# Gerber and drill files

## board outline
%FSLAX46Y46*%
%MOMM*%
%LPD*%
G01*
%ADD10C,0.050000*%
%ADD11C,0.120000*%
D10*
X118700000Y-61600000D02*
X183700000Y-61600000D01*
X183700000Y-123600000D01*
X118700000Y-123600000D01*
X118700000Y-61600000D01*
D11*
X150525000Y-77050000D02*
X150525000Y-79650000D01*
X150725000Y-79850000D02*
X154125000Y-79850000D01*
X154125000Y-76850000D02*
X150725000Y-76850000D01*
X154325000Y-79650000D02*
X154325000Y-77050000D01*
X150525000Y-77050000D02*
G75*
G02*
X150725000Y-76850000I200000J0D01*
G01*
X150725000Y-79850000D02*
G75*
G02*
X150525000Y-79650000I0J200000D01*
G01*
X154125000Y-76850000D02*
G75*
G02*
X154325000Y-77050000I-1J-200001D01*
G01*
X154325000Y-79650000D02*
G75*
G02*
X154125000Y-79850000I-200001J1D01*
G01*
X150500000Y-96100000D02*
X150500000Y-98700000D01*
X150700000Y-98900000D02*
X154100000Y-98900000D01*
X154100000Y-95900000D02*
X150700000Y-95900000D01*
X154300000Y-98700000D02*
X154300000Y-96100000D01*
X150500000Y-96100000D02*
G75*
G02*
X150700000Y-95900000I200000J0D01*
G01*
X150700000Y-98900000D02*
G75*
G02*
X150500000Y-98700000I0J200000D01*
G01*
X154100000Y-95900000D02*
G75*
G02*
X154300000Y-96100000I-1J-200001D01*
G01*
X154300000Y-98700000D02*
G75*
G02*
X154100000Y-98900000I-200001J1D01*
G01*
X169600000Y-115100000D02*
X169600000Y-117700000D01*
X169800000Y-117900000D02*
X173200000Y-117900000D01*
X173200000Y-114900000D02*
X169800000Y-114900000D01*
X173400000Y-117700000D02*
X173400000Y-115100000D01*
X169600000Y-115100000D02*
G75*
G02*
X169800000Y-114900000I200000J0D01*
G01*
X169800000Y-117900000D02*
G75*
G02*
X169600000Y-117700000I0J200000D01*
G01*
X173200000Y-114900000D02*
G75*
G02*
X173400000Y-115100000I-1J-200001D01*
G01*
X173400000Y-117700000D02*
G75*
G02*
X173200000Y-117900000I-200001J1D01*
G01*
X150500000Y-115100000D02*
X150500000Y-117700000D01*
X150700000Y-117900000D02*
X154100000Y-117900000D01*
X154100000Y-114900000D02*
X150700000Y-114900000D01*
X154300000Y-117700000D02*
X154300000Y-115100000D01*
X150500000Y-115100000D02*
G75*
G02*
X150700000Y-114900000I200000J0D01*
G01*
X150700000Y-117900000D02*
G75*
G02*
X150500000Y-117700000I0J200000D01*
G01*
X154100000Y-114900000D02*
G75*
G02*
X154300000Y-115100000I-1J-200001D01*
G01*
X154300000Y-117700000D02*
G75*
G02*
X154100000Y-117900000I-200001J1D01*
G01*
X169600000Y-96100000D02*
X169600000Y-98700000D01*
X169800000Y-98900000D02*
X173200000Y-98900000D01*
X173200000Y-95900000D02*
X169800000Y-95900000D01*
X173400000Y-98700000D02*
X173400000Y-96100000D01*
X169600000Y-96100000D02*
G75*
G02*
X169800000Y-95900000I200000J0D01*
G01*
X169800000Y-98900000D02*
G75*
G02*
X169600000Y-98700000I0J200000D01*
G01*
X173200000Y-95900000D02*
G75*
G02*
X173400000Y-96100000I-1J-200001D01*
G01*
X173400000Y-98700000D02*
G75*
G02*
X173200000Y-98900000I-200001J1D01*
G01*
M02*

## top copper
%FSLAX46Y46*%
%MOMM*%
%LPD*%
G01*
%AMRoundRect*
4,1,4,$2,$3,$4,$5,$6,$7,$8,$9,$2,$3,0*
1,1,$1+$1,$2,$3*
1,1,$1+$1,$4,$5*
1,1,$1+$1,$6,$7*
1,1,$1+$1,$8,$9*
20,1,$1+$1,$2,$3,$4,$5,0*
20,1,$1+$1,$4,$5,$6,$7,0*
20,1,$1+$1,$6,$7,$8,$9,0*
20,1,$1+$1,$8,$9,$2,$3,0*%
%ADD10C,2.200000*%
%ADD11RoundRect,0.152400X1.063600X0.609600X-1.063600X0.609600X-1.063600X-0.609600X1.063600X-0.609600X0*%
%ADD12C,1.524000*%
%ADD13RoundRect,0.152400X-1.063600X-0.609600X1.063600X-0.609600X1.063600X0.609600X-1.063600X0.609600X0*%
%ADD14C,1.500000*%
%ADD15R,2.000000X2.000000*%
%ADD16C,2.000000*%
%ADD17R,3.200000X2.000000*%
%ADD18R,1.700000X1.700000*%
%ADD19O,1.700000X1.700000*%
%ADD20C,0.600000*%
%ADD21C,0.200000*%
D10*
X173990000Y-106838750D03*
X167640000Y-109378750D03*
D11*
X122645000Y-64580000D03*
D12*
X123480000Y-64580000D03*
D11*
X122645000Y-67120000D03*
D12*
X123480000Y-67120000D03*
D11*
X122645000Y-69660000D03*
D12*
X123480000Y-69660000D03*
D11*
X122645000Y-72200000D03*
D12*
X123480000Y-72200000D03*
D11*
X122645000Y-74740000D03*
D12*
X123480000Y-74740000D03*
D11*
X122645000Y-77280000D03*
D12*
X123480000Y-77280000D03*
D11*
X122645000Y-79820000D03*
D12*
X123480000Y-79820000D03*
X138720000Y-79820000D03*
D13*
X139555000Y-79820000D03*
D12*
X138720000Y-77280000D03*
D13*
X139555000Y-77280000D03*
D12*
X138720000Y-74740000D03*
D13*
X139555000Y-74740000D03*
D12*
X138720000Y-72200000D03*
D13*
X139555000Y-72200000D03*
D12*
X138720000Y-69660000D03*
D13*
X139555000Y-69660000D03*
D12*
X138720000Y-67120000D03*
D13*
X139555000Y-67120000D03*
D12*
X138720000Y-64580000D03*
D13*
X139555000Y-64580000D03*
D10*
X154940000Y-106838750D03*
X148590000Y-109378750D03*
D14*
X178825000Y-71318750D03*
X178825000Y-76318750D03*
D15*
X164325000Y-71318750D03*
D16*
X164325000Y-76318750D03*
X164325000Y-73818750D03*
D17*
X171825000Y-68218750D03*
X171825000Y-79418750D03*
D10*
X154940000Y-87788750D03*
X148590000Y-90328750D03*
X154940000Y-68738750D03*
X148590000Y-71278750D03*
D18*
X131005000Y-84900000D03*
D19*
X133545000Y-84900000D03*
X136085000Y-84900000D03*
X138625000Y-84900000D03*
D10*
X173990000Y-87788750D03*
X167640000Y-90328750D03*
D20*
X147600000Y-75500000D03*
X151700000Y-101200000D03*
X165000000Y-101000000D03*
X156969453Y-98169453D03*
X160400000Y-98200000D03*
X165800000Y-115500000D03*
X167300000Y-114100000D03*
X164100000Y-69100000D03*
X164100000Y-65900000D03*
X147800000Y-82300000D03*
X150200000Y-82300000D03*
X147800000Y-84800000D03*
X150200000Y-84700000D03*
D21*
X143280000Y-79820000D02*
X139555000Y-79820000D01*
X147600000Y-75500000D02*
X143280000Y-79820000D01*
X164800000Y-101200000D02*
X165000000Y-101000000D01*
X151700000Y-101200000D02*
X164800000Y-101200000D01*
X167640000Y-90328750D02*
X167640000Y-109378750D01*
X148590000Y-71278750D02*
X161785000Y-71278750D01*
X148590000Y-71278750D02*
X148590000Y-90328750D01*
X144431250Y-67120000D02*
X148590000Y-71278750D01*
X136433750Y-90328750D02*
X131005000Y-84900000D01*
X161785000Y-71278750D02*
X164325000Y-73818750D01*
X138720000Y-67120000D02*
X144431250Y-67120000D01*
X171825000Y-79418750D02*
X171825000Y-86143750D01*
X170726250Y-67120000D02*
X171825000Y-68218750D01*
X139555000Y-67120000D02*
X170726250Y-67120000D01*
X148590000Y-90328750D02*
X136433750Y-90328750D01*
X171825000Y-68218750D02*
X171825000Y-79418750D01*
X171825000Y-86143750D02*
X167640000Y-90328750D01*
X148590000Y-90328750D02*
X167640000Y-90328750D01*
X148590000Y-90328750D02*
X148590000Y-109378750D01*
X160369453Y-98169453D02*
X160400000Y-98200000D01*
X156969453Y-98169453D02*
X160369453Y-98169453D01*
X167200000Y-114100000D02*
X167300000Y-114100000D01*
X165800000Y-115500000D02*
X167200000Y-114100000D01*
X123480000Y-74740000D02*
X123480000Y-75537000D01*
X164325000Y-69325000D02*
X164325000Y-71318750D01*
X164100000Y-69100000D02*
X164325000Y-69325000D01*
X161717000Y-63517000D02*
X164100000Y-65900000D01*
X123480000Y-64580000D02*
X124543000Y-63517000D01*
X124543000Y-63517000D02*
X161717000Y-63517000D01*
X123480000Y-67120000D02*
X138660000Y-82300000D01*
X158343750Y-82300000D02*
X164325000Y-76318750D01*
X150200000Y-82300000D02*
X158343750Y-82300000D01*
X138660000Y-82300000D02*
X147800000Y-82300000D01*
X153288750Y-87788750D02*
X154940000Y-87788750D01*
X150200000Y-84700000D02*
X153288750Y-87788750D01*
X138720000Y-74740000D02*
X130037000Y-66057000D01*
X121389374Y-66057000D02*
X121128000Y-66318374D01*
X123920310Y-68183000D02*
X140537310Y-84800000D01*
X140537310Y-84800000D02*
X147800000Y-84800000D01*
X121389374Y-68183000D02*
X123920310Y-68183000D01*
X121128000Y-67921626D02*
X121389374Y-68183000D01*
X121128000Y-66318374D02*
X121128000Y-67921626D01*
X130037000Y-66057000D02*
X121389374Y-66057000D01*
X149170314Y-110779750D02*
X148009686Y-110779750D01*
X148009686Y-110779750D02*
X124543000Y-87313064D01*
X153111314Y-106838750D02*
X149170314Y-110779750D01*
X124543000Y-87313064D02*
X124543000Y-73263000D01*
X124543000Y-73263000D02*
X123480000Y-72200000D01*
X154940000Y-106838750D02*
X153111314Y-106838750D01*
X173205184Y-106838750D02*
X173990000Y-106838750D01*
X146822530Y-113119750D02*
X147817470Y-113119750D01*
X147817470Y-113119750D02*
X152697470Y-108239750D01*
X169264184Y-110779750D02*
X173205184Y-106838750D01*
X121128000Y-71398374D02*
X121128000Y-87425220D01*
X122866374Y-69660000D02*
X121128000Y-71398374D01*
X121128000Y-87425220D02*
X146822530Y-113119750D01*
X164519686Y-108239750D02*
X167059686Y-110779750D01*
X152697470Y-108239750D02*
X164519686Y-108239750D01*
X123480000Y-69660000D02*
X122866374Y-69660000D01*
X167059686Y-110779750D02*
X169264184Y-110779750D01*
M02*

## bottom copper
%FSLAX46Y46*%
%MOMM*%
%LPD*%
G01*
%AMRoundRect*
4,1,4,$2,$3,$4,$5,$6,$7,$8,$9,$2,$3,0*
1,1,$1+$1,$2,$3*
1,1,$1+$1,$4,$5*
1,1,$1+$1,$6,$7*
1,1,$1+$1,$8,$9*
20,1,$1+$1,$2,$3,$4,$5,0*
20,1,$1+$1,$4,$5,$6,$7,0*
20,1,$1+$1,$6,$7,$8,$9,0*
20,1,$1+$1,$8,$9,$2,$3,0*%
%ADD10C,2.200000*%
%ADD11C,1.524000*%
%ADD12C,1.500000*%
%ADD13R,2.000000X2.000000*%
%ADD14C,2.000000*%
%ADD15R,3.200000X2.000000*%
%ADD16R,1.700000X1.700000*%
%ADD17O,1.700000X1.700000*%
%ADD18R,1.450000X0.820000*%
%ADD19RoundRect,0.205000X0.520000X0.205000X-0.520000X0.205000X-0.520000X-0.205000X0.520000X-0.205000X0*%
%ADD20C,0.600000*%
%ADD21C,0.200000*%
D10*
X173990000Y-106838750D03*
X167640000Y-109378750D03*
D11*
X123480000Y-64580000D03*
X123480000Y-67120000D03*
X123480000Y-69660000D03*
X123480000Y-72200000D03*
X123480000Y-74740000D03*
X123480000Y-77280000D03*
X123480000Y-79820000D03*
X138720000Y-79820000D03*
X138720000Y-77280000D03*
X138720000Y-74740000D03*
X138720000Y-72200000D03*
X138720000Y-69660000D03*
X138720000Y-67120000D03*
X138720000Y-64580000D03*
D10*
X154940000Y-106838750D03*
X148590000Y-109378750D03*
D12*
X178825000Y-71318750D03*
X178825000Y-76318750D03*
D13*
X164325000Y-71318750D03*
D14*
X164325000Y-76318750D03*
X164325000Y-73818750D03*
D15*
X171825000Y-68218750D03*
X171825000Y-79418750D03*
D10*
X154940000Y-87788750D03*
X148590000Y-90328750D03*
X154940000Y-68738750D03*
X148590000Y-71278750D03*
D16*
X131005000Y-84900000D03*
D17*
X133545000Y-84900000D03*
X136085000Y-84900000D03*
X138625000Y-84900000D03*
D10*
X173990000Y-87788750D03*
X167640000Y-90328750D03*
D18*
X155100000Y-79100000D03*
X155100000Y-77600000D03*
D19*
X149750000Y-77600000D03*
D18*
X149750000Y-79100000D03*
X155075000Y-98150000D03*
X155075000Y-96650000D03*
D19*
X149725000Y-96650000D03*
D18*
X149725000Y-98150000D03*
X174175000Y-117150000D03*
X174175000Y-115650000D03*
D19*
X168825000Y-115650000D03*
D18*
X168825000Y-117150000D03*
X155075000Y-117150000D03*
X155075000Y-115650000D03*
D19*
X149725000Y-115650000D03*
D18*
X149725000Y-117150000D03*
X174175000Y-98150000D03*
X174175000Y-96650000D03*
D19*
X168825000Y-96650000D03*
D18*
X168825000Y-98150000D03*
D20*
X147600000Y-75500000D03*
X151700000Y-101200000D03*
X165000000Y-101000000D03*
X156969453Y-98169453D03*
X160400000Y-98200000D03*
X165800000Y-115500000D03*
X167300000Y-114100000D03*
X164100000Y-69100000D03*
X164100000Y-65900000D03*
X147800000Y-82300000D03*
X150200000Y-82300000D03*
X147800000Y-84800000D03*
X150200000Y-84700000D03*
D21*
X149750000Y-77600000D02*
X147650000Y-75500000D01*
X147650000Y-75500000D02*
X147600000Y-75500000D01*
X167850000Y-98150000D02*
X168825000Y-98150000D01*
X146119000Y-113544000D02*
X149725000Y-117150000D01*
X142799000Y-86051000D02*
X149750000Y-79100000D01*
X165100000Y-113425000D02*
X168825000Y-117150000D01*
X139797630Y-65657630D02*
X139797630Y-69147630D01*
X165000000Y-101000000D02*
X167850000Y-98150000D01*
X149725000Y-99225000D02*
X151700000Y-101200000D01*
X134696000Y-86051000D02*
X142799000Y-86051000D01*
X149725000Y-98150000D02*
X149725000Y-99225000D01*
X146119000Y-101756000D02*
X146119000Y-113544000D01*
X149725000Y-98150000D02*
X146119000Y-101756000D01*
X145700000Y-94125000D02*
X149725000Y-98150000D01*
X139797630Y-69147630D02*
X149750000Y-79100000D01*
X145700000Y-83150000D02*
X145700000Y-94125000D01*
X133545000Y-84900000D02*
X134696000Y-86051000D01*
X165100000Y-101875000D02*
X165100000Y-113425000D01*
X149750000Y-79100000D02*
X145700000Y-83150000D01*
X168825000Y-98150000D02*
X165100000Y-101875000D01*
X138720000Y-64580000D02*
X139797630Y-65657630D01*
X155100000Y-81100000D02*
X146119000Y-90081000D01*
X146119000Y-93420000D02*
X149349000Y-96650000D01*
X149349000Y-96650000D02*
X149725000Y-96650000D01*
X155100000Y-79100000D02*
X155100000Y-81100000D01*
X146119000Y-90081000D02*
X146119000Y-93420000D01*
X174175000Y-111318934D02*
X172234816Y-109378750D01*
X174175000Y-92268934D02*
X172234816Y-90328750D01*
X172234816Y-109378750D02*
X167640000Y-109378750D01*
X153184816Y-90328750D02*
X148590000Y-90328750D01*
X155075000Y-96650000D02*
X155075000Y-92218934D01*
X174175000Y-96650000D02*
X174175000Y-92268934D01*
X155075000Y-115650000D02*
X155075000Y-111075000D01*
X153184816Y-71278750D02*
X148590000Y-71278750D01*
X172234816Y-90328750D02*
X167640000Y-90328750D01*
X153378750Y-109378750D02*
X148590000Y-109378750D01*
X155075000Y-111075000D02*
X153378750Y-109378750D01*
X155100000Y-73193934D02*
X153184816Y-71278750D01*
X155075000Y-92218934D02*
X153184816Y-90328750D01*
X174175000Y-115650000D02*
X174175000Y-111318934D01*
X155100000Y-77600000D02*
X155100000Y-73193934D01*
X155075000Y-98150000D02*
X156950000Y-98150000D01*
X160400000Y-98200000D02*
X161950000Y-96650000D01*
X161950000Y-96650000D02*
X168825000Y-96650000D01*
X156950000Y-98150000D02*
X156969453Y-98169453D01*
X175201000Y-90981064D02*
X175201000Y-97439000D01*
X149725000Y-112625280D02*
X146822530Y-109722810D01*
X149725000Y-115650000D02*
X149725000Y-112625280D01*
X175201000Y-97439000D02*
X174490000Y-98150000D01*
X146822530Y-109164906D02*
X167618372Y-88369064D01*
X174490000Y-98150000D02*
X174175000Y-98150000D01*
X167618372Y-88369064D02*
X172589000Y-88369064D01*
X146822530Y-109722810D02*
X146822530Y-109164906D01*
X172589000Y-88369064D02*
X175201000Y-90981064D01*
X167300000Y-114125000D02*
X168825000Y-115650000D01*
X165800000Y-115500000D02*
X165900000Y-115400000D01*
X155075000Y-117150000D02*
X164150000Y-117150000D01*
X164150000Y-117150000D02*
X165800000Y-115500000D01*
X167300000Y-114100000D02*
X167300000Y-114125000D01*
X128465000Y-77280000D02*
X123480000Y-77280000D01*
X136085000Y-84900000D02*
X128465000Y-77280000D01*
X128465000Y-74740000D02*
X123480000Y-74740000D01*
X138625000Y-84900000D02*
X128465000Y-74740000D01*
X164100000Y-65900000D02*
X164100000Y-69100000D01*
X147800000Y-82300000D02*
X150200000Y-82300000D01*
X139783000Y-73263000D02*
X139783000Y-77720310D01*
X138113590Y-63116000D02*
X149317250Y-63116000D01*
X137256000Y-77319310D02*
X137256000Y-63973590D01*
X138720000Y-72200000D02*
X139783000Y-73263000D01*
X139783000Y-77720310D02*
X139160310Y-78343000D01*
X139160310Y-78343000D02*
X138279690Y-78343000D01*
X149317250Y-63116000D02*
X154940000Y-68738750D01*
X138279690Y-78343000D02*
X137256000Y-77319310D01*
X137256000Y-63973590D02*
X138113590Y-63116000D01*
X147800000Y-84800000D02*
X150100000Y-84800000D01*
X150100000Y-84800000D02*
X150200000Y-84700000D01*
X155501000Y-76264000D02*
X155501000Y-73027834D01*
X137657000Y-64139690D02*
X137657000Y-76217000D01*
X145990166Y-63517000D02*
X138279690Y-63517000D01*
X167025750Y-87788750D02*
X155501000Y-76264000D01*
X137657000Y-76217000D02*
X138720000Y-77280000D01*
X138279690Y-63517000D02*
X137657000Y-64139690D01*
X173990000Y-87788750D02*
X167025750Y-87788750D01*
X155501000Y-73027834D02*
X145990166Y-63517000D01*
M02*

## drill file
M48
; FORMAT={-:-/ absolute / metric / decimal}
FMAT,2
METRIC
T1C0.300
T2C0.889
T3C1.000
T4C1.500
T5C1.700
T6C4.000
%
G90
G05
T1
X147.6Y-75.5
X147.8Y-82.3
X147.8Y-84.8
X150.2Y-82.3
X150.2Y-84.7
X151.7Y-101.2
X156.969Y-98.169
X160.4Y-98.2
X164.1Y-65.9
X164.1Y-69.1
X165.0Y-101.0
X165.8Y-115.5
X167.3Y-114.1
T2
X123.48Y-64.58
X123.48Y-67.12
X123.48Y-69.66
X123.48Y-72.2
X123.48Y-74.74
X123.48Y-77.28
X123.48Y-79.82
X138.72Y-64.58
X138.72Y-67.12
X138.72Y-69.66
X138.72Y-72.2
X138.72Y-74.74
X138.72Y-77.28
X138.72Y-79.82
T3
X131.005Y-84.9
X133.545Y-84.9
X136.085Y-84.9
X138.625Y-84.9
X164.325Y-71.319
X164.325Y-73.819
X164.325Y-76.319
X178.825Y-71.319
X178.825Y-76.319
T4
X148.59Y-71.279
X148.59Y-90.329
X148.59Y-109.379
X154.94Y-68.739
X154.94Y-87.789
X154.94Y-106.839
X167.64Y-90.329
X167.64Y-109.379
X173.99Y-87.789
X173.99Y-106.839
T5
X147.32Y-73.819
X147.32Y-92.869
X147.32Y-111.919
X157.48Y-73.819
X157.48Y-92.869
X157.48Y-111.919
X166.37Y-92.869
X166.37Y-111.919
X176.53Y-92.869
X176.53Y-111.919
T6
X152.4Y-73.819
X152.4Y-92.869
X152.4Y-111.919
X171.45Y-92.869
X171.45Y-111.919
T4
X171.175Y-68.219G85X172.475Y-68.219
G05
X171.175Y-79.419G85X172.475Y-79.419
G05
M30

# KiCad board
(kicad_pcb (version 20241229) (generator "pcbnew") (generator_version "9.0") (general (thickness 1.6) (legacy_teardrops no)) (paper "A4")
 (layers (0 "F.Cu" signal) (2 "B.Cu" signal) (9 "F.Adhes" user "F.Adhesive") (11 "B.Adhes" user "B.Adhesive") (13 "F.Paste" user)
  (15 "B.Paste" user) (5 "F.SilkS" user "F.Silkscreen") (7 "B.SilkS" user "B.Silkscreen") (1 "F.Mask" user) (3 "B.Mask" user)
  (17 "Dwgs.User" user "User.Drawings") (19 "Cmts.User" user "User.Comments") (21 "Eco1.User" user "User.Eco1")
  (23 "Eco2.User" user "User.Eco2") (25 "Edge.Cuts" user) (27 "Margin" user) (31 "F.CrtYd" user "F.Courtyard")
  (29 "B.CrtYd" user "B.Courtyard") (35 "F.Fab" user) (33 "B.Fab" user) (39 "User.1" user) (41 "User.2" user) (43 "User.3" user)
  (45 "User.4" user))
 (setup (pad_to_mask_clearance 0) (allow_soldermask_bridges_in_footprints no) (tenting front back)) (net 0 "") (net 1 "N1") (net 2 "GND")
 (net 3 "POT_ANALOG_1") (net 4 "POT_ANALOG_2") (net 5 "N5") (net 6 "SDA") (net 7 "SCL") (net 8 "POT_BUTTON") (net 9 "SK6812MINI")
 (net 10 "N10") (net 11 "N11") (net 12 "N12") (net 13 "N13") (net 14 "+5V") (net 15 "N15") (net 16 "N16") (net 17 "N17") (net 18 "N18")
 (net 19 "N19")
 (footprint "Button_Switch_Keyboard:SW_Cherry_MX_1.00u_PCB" (layer "F.Cu") (at 173.99 106.83875)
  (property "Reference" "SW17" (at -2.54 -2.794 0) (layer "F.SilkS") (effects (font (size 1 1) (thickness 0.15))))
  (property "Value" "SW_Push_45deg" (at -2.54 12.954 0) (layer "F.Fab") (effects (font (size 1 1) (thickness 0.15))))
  (pad "" np_thru_hole circle (at -7.62 5.08) (size 1.7 1.7) (drill 1.7) (layers "*.Cu" "*.Mask"))
  (pad "" np_thru_hole circle (at -2.54 5.08) (size 4 4) (drill 4) (layers "*.Cu" "*.Mask"))
  (pad "" np_thru_hole circle (at 2.54 5.08) (size 1.7 1.7) (drill 1.7) (layers "*.Cu" "*.Mask"))
  (pad "1" thru_hole circle (at 0 0) (size 2.2 2.2) (drill 1.5) (layers "*.Cu" "*.Mask") (remove_unused_layers no) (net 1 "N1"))
  (pad "2" thru_hole circle (at -6.35 2.54) (size 2.2 2.2) (drill 1.5) (layers "*.Cu" "*.Mask") (remove_unused_layers no) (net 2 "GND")))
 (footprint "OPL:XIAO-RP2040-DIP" (layer "F.Cu") (at 131.1 72.2)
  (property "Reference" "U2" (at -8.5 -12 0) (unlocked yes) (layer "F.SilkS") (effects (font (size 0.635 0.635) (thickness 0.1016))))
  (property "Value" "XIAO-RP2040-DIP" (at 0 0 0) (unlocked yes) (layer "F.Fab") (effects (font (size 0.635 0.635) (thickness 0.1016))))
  (pad "1" smd roundrect (at -8.455 -7.62 180) (size 2.432 1.524) (layers "F.Cu" "F.Mask") (roundrect_rratio 0.1) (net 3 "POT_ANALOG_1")
   (thermal_bridge_angle 45))
  (pad "1" thru_hole circle (at -7.62 -7.62 180) (size 1.524 1.524) (drill 0.889) (layers "*.Cu" "*.Mask") (remove_unused_layers no)
   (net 3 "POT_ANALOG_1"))
  (pad "2" smd roundrect (at -8.455 -5.08 180) (size 2.432 1.524) (layers "F.Cu" "F.Mask") (roundrect_rratio 0.1) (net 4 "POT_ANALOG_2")
   (thermal_bridge_angle 45))
  (pad "2" thru_hole circle (at -7.62 -5.08 180) (size 1.524 1.524) (drill 0.889) (layers "*.Cu" "*.Mask") (remove_unused_layers no)
   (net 4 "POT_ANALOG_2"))
  (pad "3" smd roundrect (at -8.455 -2.54 180) (size 2.432 1.524) (layers "F.Cu" "F.Mask") (roundrect_rratio 0.1) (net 1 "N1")
   (thermal_bridge_angle 45))
  (pad "3" thru_hole circle (at -7.62 -2.54 180) (size 1.524 1.524) (drill 0.889) (layers "*.Cu" "*.Mask") (remove_unused_layers no)
   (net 1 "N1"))
  (pad "4" smd roundrect (at -8.455 0 180) (size 2.432 1.524) (layers "F.Cu" "F.Mask") (roundrect_rratio 0.1) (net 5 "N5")
   (thermal_bridge_angle 45))
  (pad "4" thru_hole circle (at -7.62 0 180) (size 1.524 1.524) (drill 0.889) (layers "*.Cu" "*.Mask") (remove_unused_layers no)
   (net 5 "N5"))
  (pad "5" smd roundrect (at -8.455 2.54 180) (size 2.432 1.524) (layers "F.Cu" "F.Mask") (roundrect_rratio 0.1) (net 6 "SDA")
   (thermal_bridge_angle 45))
  (pad "5" thru_hole circle (at -7.62 2.54 180) (size 1.524 1.524) (drill 0.889) (layers "*.Cu" "*.Mask") (remove_unused_layers no)
   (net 6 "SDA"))
  (pad "6" smd roundrect (at -8.455 5.08 180) (size 2.432 1.524) (layers "F.Cu" "F.Mask") (roundrect_rratio 0.1) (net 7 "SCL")
   (thermal_bridge_angle 45))
  (pad "6" thru_hole circle (at -7.62 5.08 180) (size 1.524 1.524) (drill 0.889) (layers "*.Cu" "*.Mask") (remove_unused_layers no)
   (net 7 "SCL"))
  (pad "7" smd roundrect (at -8.455 7.62 180) (size 2.432 1.524) (layers "F.Cu" "F.Mask") (roundrect_rratio 0.1) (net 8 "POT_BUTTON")
   (thermal_bridge_angle 45))
  (pad "7" thru_hole circle (at -7.62 7.62 180) (size 1.524 1.524) (drill 0.889) (layers "*.Cu" "*.Mask") (remove_unused_layers no)
   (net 8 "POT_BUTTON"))
  (pad "8" thru_hole circle (at 7.62 7.62) (size 1.524 1.524) (drill 0.889) (layers "*.Cu" "*.Mask") (remove_unused_layers no)
   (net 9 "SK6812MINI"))
  (pad "8" smd roundrect (at 8.455 7.62) (size 2.432 1.524) (layers "F.Cu" "F.Mask") (roundrect_rratio 0.1) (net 9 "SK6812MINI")
   (thermal_bridge_angle 45))
  (pad "9" thru_hole circle (at 7.62 5.08) (size 1.524 1.524) (drill 0.889) (layers "*.Cu" "*.Mask") (remove_unused_layers no)
   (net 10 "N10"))
  (pad "9" smd roundrect (at 8.455 5.08) (size 2.432 1.524) (layers "F.Cu" "F.Mask") (roundrect_rratio 0.1) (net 10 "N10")
   (thermal_bridge_angle 45))
  (pad "10" thru_hole circle (at 7.62 2.54) (size 1.524 1.524) (drill 0.889) (layers "*.Cu" "*.Mask") (remove_unused_layers no)
   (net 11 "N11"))
  (pad "10" smd roundrect (at 8.455 2.54) (size 2.432 1.524) (layers "F.Cu" "F.Mask") (roundrect_rratio 0.1) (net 11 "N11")
   (thermal_bridge_angle 45))
  (pad "11" thru_hole circle (at 7.62 0) (size 1.524 1.524) (drill 0.889) (layers "*.Cu" "*.Mask") (remove_unused_layers no) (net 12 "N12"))
  (pad "11" smd roundrect (at 8.455 0) (size 2.432 1.524) (layers "F.Cu" "F.Mask") (roundrect_rratio 0.1) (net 12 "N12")
   (thermal_bridge_angle 45))
  (pad "12" thru_hole circle (at 7.62 -2.54) (size 1.524 1.524) (drill 0.889) (layers "*.Cu" "*.Mask") (remove_unused_layers no)
   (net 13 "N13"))
  (pad "12" smd roundrect (at 8.455 -2.54) (size 2.432 1.524) (layers "F.Cu" "F.Mask") (roundrect_rratio 0.1) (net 13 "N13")
   (thermal_bridge_angle 45))
  (pad "13" thru_hole circle (at 7.62 -5.08) (size 1.524 1.524) (drill 0.889) (layers "*.Cu" "*.Mask") (remove_unused_layers no)
   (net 2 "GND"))
  (pad "13" smd roundrect (at 8.455 -5.08) (size 2.432 1.524) (layers "F.Cu" "F.Mask") (roundrect_rratio 0.1) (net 2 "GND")
   (thermal_bridge_angle 45))
  (pad "14" thru_hole circle (at 7.62 -7.62) (size 1.524 1.524) (drill 0.889) (layers "*.Cu" "*.Mask") (remove_unused_layers no)
   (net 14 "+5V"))
  (pad "14" smd roundrect (at 8.455 -7.62) (size 2.432 1.524) (layers "F.Cu" "F.Mask") (roundrect_rratio 0.1) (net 14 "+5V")
   (thermal_bridge_angle 45)))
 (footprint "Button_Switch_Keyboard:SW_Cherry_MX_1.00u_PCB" (layer "F.Cu") (at 154.94 106.83875)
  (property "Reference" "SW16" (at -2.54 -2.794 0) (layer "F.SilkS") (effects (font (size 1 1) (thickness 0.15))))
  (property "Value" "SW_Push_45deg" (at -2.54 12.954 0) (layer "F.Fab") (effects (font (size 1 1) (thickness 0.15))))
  (pad "" np_thru_hole circle (at -7.62 5.08) (size 1.7 1.7) (drill 1.7) (layers "*.Cu" "*.Mask"))
  (pad "" np_thru_hole circle (at -2.54 5.08) (size 4 4) (drill 4) (layers "*.Cu" "*.Mask"))
  (pad "" np_thru_hole circle (at 2.54 5.08) (size 1.7 1.7) (drill 1.7) (layers "*.Cu" "*.Mask"))
  (pad "1" thru_hole circle (at 0 0) (size 2.2 2.2) (drill 1.5) (layers "*.Cu" "*.Mask") (remove_unused_layers no) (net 5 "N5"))
  (pad "2" thru_hole circle (at -6.35 2.54) (size 2.2 2.2) (drill 1.5) (layers "*.Cu" "*.Mask") (remove_unused_layers no) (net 2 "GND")))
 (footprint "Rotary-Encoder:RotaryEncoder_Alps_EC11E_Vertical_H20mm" (layer "F.Cu") (at 164.325 71.31875)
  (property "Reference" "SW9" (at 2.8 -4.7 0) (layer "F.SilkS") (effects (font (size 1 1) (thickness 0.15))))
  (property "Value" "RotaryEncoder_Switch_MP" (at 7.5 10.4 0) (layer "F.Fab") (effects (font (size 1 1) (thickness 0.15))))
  (pad "" thru_hole circle (at 14.5 0) (size 1.5 1.5) (drill 1) (layers "*.Cu" "*.Mask") (remove_unused_layers no))
  (pad "" thru_hole circle (at 14.5 5) (size 1.5 1.5) (drill 1) (layers "*.Cu" "*.Mask") (remove_unused_layers no))
  (pad "A" thru_hole rect (at 0 0) (size 2 2) (drill 1) (layers "*.Cu" "*.Mask") (remove_unused_layers no) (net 3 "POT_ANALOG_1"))
  (pad "B" thru_hole circle (at 0 5) (size 2 2) (drill 1) (layers "*.Cu" "*.Mask") (remove_unused_layers no) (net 4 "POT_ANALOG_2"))
  (pad "C" thru_hole circle (at 0 2.5) (size 2 2) (drill 1) (layers "*.Cu" "*.Mask") (remove_unused_layers no) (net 2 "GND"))
  (pad "MP" thru_hole rect (at 7.5 -3.1) (size 3.2 2) (drill oval 2.8 1.5) (layers "*.Cu" "*.Mask") (remove_unused_layers no) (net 2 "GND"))
  (pad "MP" thru_hole rect (at 7.5 8.1) (size 3.2 2) (drill oval 2.8 1.5) (layers "*.Cu" "*.Mask") (remove_unused_layers no) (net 2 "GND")))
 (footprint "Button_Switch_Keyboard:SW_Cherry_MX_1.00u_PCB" (layer "F.Cu") (at 154.94 87.78875)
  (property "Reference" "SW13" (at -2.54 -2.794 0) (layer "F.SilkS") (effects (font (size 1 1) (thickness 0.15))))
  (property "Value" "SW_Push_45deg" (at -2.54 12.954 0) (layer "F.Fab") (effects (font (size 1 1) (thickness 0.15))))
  (pad "" np_thru_hole circle (at -7.62 5.08) (size 1.7 1.7) (drill 1.7) (layers "*.Cu" "*.Mask"))
  (pad "" np_thru_hole circle (at -2.54 5.08) (size 4 4) (drill 4) (layers "*.Cu" "*.Mask"))
  (pad "" np_thru_hole circle (at 2.54 5.08) (size 1.7 1.7) (drill 1.7) (layers "*.Cu" "*.Mask"))
  (pad "1" thru_hole circle (at 0 0) (size 2.2 2.2) (drill 1.5) (layers "*.Cu" "*.Mask") (remove_unused_layers no) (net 11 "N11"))
  (pad "2" thru_hole circle (at -6.35 2.54) (size 2.2 2.2) (drill 1.5) (layers "*.Cu" "*.Mask") (remove_unused_layers no) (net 2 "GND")))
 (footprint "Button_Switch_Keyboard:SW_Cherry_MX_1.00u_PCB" (layer "F.Cu") (at 154.94 68.73875)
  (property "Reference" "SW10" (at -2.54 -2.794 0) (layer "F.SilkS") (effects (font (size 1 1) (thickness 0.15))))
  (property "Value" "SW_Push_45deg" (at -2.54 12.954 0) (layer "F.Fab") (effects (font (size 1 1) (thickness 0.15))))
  (pad "" np_thru_hole circle (at -7.62 5.08) (size 1.7 1.7) (drill 1.7) (layers "*.Cu" "*.Mask"))
  (pad "" np_thru_hole circle (at -2.54 5.08) (size 4 4) (drill 4) (layers "*.Cu" "*.Mask"))
  (pad "" np_thru_hole circle (at 2.54 5.08) (size 1.7 1.7) (drill 1.7) (layers "*.Cu" "*.Mask"))
  (pad "1" thru_hole circle (at 0 0) (size 2.2 2.2) (drill 1.5) (layers "*.Cu" "*.Mask") (remove_unused_layers no) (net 12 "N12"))
  (pad "2" thru_hole circle (at -6.35 2.54) (size 2.2 2.2) (drill 1.5) (layers "*.Cu" "*.Mask") (remove_unused_layers no) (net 2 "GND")))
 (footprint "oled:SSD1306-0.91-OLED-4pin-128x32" (layer "F.Cu") (at 128.815 121.4 90)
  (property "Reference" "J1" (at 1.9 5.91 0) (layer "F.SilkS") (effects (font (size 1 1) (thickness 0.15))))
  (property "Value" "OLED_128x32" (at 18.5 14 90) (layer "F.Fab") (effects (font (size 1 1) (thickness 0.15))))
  (pad "1" thru_hole rect (at 36.5 2.19 90) (size 1.7 1.7) (drill 1) (layers "*.Cu" "*.Mask") (remove_unused_layers no) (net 2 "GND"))
  (pad "2" thru_hole oval (at 36.5 4.73 90) (size 1.7 1.7) (drill 1) (layers "*.Cu" "*.Mask") (remove_unused_layers no) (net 14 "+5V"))
  (pad "3" thru_hole oval (at 36.5 7.27 90) (size 1.7 1.7) (drill 1) (layers "*.Cu" "*.Mask") (remove_unused_layers no) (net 7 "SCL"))
  (pad "4" thru_hole oval (at 36.5 9.81 90) (size 1.7 1.7) (drill 1) (layers "*.Cu" "*.Mask") (remove_unused_layers no) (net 6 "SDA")))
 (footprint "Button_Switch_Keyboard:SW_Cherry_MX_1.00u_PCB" (layer "F.Cu") (at 173.99 87.78875)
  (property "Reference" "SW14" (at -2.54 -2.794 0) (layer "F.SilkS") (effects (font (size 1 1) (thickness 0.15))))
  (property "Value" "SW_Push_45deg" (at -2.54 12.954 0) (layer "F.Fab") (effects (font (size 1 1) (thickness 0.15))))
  (pad "" np_thru_hole circle (at -7.62 5.08) (size 1.7 1.7) (drill 1.7) (layers "*.Cu" "*.Mask"))
  (pad "" np_thru_hole circle (at -2.54 5.08) (size 4 4) (drill 4) (layers "*.Cu" "*.Mask"))
  (pad "" np_thru_hole circle (at 2.54 5.08) (size 1.7 1.7) (drill 1.7) (layers "*.Cu" "*.Mask"))
  (pad "1" thru_hole circle (at 0 0) (size 2.2 2.2) (drill 1.5) (layers "*.Cu" "*.Mask") (remove_unused_layers no) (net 10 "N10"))
  (pad "2" thru_hole circle (at -6.35 2.54) (size 2.2 2.2) (drill 1.5) (layers "*.Cu" "*.Mask") (remove_unused_layers no) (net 2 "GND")))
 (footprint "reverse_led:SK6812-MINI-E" (layer "B.Cu") (at 152.425 78.35 180)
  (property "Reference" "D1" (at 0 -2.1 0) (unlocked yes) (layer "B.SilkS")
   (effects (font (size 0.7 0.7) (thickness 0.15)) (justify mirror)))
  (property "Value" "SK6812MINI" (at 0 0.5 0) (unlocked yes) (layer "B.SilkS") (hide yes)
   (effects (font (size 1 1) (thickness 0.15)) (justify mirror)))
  (fp_line (start 1.9 1.3) (end 1.9 -1.3) (stroke (width 0.12) (type solid)) (layer "Edge.Cuts"))
  (fp_line (start 1.7 -1.5) (end -1.7 -1.5) (stroke (width 0.12) (type solid)) (layer "Edge.Cuts"))
  (fp_line (start -1.7 1.5) (end 1.7 1.5) (stroke (width 0.12) (type solid)) (layer "Edge.Cuts"))
  (fp_line (start -1.9 -1.3) (end -1.9 1.3) (stroke (width 0.12) (type solid)) (layer "Edge.Cuts"))
  (fp_arc (start 1.9 1.3) (mid 1.841421 1.441421) (end 1.7 1.5) (stroke (width 0.12) (type solid)) (layer "Edge.Cuts"))
  (fp_arc (start 1.7 -1.5) (mid 1.841421 -1.441421) (end 1.9 -1.3) (stroke (width 0.12) (type solid)) (layer "Edge.Cuts"))
  (fp_arc (start -1.7 1.5) (mid -1.841421 1.441421) (end -1.9 1.3) (stroke (width 0.12) (type solid)) (layer "Edge.Cuts"))
  (fp_arc (start -1.9 -1.3) (mid -1.841421 -1.441421) (end -1.7 -1.5) (stroke (width 0.12) (type solid)) (layer "Edge.Cuts"))
  (pad "1" smd rect (at -2.675 -0.75 180) (size 1.45 0.82) (layers "B.Cu" "B.Mask" "B.Paste") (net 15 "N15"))
  (pad "2" smd rect (at -2.675 0.75 180) (size 1.45 0.82) (layers "B.Cu" "B.Mask" "B.Paste") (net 2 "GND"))
  (pad "3" smd roundrect (at 2.675 0.75 180) (size 1.45 0.82) (layers "B.Cu" "B.Mask" "B.Paste") (roundrect_rratio 0.25)
   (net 9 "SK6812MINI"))
  (pad "4" smd rect (at 2.675 -0.75 180) (size 1.45 0.82) (layers "B.Cu" "B.Mask" "B.Paste") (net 14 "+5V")))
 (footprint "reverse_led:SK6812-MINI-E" (layer "B.Cu") (at 152.4 97.4 180)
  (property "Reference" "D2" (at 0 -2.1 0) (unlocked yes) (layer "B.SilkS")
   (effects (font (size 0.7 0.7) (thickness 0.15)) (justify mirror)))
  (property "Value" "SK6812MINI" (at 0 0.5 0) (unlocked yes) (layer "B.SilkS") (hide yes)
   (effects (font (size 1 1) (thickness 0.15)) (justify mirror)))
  (fp_line (start 1.9 1.3) (end 1.9 -1.3) (stroke (width 0.12) (type solid)) (layer "Edge.Cuts"))
  (fp_line (start 1.7 -1.5) (end -1.7 -1.5) (stroke (width 0.12) (type solid)) (layer "Edge.Cuts"))
  (fp_line (start -1.7 1.5) (end 1.7 1.5) (stroke (width 0.12) (type solid)) (layer "Edge.Cuts"))
  (fp_line (start -1.9 -1.3) (end -1.9 1.3) (stroke (width 0.12) (type solid)) (layer "Edge.Cuts"))
  (fp_arc (start 1.9 1.3) (mid 1.841421 1.441421) (end 1.7 1.5) (stroke (width 0.12) (type solid)) (layer "Edge.Cuts"))
  (fp_arc (start 1.7 -1.5) (mid 1.841421 -1.441421) (end 1.9 -1.3) (stroke (width 0.12) (type solid)) (layer "Edge.Cuts"))
  (fp_arc (start -1.7 1.5) (mid -1.841421 1.441421) (end -1.9 1.3) (stroke (width 0.12) (type solid)) (layer "Edge.Cuts"))
  (fp_arc (start -1.9 -1.3) (mid -1.841421 -1.441421) (end -1.7 -1.5) (stroke (width 0.12) (type solid)) (layer "Edge.Cuts"))
  (pad "1" smd rect (at -2.675 -0.75 180) (size 1.45 0.82) (layers "B.Cu" "B.Mask" "B.Paste") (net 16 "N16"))
  (pad "2" smd rect (at -2.675 0.75 180) (size 1.45 0.82) (layers "B.Cu" "B.Mask" "B.Paste") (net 2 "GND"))
  (pad "3" smd roundrect (at 2.675 0.75 180) (size 1.45 0.82) (layers "B.Cu" "B.Mask" "B.Paste") (roundrect_rratio 0.25) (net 15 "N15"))
  (pad "4" smd rect (at 2.675 -0.75 180) (size 1.45 0.82) (layers "B.Cu" "B.Mask" "B.Paste") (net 14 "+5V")))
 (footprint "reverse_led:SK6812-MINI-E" (layer "B.Cu") (at 171.5 116.4 180)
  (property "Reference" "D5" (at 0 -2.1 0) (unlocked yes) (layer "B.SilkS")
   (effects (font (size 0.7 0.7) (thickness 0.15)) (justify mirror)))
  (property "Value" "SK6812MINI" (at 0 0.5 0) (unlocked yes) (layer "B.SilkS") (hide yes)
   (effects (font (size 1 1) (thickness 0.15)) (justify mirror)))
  (fp_line (start 1.9 1.3) (end 1.9 -1.3) (stroke (width 0.12) (type solid)) (layer "Edge.Cuts"))
  (fp_line (start 1.7 -1.5) (end -1.7 -1.5) (stroke (width 0.12) (type solid)) (layer "Edge.Cuts"))
  (fp_line (start -1.7 1.5) (end 1.7 1.5) (stroke (width 0.12) (type solid)) (layer "Edge.Cuts"))
  (fp_line (start -1.9 -1.3) (end -1.9 1.3) (stroke (width 0.12) (type solid)) (layer "Edge.Cuts"))
  (fp_arc (start 1.9 1.3) (mid 1.841421 1.441421) (end 1.7 1.5) (stroke (width 0.12) (type solid)) (layer "Edge.Cuts"))
  (fp_arc (start 1.7 -1.5) (mid 1.841421 -1.441421) (end 1.9 -1.3) (stroke (width 0.12) (type solid)) (layer "Edge.Cuts"))
  (fp_arc (start -1.7 1.5) (mid -1.841421 1.441421) (end -1.9 1.3) (stroke (width 0.12) (type solid)) (layer "Edge.Cuts"))
  (fp_arc (start -1.9 -1.3) (mid -1.841421 -1.441421) (end -1.7 -1.5) (stroke (width 0.12) (type solid)) (layer "Edge.Cuts"))
  (pad "1" smd rect (at -2.675 -0.75 180) (size 1.45 0.82) (layers "B.Cu" "B.Mask" "B.Paste") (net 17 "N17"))
  (pad "2" smd rect (at -2.675 0.75 180) (size 1.45 0.82) (layers "B.Cu" "B.Mask" "B.Paste") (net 2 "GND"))
  (pad "3" smd roundrect (at 2.675 0.75 180) (size 1.45 0.82) (layers "B.Cu" "B.Mask" "B.Paste") (roundrect_rratio 0.25) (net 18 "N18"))
  (pad "4" smd rect (at 2.675 -0.75 180) (size 1.45 0.82) (layers "B.Cu" "B.Mask" "B.Paste") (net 14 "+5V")))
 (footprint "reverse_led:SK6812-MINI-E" (layer "B.Cu") (at 152.4 116.4 180)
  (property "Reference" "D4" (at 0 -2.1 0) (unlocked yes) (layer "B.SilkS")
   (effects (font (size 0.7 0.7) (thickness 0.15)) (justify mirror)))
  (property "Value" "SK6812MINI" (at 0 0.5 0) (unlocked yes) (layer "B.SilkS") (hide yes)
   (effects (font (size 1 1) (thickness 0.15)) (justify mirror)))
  (fp_line (start 1.9 1.3) (end 1.9 -1.3) (stroke (width 0.12) (type solid)) (layer "Edge.Cuts"))
  (fp_line (start 1.7 -1.5) (end -1.7 -1.5) (stroke (width 0.12) (type solid)) (layer "Edge.Cuts"))
  (fp_line (start -1.7 1.5) (end 1.7 1.5) (stroke (width 0.12) (type solid)) (layer "Edge.Cuts"))
  (fp_line (start -1.9 -1.3) (end -1.9 1.3) (stroke (width 0.12) (type solid)) (layer "Edge.Cuts"))
  (fp_arc (start 1.9 1.3) (mid 1.841421 1.441421) (end 1.7 1.5) (stroke (width 0.12) (type solid)) (layer "Edge.Cuts"))
  (fp_arc (start 1.7 -1.5) (mid 1.841421 -1.441421) (end 1.9 -1.3) (stroke (width 0.12) (type solid)) (layer "Edge.Cuts"))
  (fp_arc (start -1.7 1.5) (mid -1.841421 1.441421) (end -1.9 1.3) (stroke (width 0.12) (type solid)) (layer "Edge.Cuts"))
  (fp_arc (start -1.9 -1.3) (mid -1.841421 -1.441421) (end -1.7 -1.5) (stroke (width 0.12) (type solid)) (layer "Edge.Cuts"))
  (pad "1" smd rect (at -2.675 -0.75 180) (size 1.45 0.82) (layers "B.Cu" "B.Mask" "B.Paste") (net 18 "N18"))
  (pad "2" smd rect (at -2.675 0.75 180) (size 1.45 0.82) (layers "B.Cu" "B.Mask" "B.Paste") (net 2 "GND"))
  (pad "3" smd roundrect (at 2.675 0.75 180) (size 1.45 0.82) (layers "B.Cu" "B.Mask" "B.Paste") (roundrect_rratio 0.25) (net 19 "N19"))
  (pad "4" smd rect (at 2.675 -0.75 180) (size 1.45 0.82) (layers "B.Cu" "B.Mask" "B.Paste") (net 14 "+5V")))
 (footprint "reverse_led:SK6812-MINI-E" (layer "B.Cu") (at 171.5 97.4 180)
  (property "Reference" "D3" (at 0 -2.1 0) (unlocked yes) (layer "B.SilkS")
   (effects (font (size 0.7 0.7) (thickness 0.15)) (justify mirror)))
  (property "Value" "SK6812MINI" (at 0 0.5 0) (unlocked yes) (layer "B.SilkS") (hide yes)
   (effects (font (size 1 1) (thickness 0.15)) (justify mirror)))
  (fp_line (start 1.9 1.3) (end 1.9 -1.3) (stroke (width 0.12) (type solid)) (layer "Edge.Cuts"))
  (fp_line (start 1.7 -1.5) (end -1.7 -1.5) (stroke (width 0.12) (type solid)) (layer "Edge.Cuts"))
  (fp_line (start -1.7 1.5) (end 1.7 1.5) (stroke (width 0.12) (type solid)) (layer "Edge.Cuts"))
  (fp_line (start -1.9 -1.3) (end -1.9 1.3) (stroke (width 0.12) (type solid)) (layer "Edge.Cuts"))
  (fp_arc (start 1.9 1.3) (mid 1.841421 1.441421) (end 1.7 1.5) (stroke (width 0.12) (type solid)) (layer "Edge.Cuts"))
  (fp_arc (start 1.7 -1.5) (mid 1.841421 -1.441421) (end 1.9 -1.3) (stroke (width 0.12) (type solid)) (layer "Edge.Cuts"))
  (fp_arc (start -1.7 1.5) (mid -1.841421 1.441421) (end -1.9 1.3) (stroke (width 0.12) (type solid)) (layer "Edge.Cuts"))
  (fp_arc (start -1.9 -1.3) (mid -1.841421 -1.441421) (end -1.7 -1.5) (stroke (width 0.12) (type solid)) (layer "Edge.Cuts"))
  (pad "1" smd rect (at -2.675 -0.75 180) (size 1.45 0.82) (layers "B.Cu" "B.Mask" "B.Paste") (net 19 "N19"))
  (pad "2" smd rect (at -2.675 0.75 180) (size 1.45 0.82) (layers "B.Cu" "B.Mask" "B.Paste") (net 2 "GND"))
  (pad "3" smd roundrect (at 2.675 0.75 180) (size 1.45 0.82) (layers "B.Cu" "B.Mask" "B.Paste") (roundrect_rratio 0.25) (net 16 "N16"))
  (pad "4" smd rect (at 2.675 -0.75 180) (size 1.45 0.82) (layers "B.Cu" "B.Mask" "B.Paste") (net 14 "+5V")))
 (gr_rect (start 118.7 61.6) (end 183.7 123.6) (stroke (width 0.05) (type solid)) (fill no) (layer "Edge.Cuts"))
 (segment (start 143.28 79.82) (end 139.555 79.82) (width 0.2) (layer "F.Cu") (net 9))
 (segment (start 147.6 75.5) (end 143.28 79.82) (width 0.2) (layer "F.Cu") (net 9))
 (via (at 147.6 75.5) (size 0.6) (drill 0.3) (layers "F.Cu" "B.Cu") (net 9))
 (segment (start 149.75 77.6) (end 147.65 75.5) (width 0.2) (layer "B.Cu") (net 9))
 (segment (start 147.65 75.5) (end 147.6 75.5) (width 0.2) (layer "B.Cu") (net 9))
 (segment (start 164.8 101.2) (end 165 101) (width 0.2) (layer "F.Cu") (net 14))
 (segment (start 151.7 101.2) (end 164.8 101.2) (width 0.2) (layer "F.Cu") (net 14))
 (via (at 151.7 101.2) (size 0.6) (drill 0.3) (layers "F.Cu" "B.Cu") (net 14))
 (via (at 165 101) (size 0.6) (drill 0.3) (layers "F.Cu" "B.Cu") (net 14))
 (segment (start 167.85 98.15) (end 168.825 98.15) (width 0.2) (layer "B.Cu") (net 14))
 (segment (start 146.119 113.544) (end 149.725 117.15) (width 0.2) (layer "B.Cu") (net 14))
 (segment (start 142.799 86.051) (end 149.75 79.1) (width 0.2) (layer "B.Cu") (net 14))
 (segment (start 165.1 113.425) (end 168.825 117.15) (width 0.2) (layer "B.Cu") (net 14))
 (segment (start 139.79763 65.65763) (end 139.79763 69.14763) (width 0.2) (layer "B.Cu") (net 14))
 (segment (start 165 101) (end 167.85 98.15) (width 0.2) (layer "B.Cu") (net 14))
 (segment (start 149.725 99.225) (end 151.7 101.2) (width 0.2) (layer "B.Cu") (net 14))
 (segment (start 134.696 86.051) (end 142.799 86.051) (width 0.2) (layer "B.Cu") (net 14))
 (segment (start 149.725 98.15) (end 149.725 99.225) (width 0.2) (layer "B.Cu") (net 14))
 (segment (start 146.119 101.756) (end 146.119 113.544) (width 0.2) (layer "B.Cu") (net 14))
 (segment (start 149.725 98.15) (end 146.119 101.756) (width 0.2) (layer "B.Cu") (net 14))
 (segment (start 145.7 94.125) (end 149.725 98.15) (width 0.2) (layer "B.Cu") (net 14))
 (segment (start 139.79763 69.14763) (end 149.75 79.1) (width 0.2) (layer "B.Cu") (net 14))
 (segment (start 145.7 83.15) (end 145.7 94.125) (width 0.2) (layer "B.Cu") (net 14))
 (segment (start 133.545 84.9) (end 134.696 86.051) (width 0.2) (layer "B.Cu") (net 14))
 (segment (start 165.1 101.875) (end 165.1 113.425) (width 0.2) (layer "B.Cu") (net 14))
 (segment (start 149.75 79.1) (end 145.7 83.15) (width 0.2) (layer "B.Cu") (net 14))
 (segment (start 168.825 98.15) (end 165.1 101.875) (width 0.2) (layer "B.Cu") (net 14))
 (segment (start 138.72 64.58) (end 139.79763 65.65763) (width 0.2) (layer "B.Cu") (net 14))
 (segment (start 155.1 81.1) (end 146.119 90.081) (width 0.2) (layer "B.Cu") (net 15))
 (segment (start 146.119 93.42) (end 149.349 96.65) (width 0.2) (layer "B.Cu") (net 15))
 (segment (start 149.349 96.65) (end 149.725 96.65) (width 0.2) (layer "B.Cu") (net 15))
 (segment (start 155.1 79.1) (end 155.1 81.1) (width 0.2) (layer "B.Cu") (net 15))
 (segment (start 146.119 90.081) (end 146.119 93.42) (width 0.2) (layer "B.Cu") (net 15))
 (segment (start 167.64 90.32875) (end 167.64 109.37875) (width 0.2) (layer "F.Cu") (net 2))
 (segment (start 148.59 71.27875) (end 161.785 71.27875) (width 0.2) (layer "F.Cu") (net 2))
 (segment (start 148.59 71.27875) (end 148.59 90.32875) (width 0.2) (layer "F.Cu") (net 2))
 (segment (start 144.43125 67.12) (end 148.59 71.27875) (width 0.2) (layer "F.Cu") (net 2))
 (segment (start 136.43375 90.32875) (end 131.005 84.9) (width 0.2) (layer "F.Cu") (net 2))
 (segment (start 161.785 71.27875) (end 164.325 73.81875) (width 0.2) (layer "F.Cu") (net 2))
 (segment (start 138.72 67.12) (end 144.43125 67.12) (width 0.2) (layer "F.Cu") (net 2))
 (segment (start 171.825 79.41875) (end 171.825 86.14375) (width 0.2) (layer "F.Cu") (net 2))
 (segment (start 170.72625 67.12) (end 171.825 68.21875) (width 0.2) (layer "F.Cu") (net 2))
 (segment (start 139.555 67.12) (end 170.72625 67.12) (width 0.2) (layer "F.Cu") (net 2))
 (segment (start 148.59 90.32875) (end 136.43375 90.32875) (width 0.2) (layer "F.Cu") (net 2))
 (segment (start 171.825 68.21875) (end 171.825 79.41875) (width 0.2) (layer "F.Cu") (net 2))
 (segment (start 171.825 86.14375) (end 167.64 90.32875) (width 0.2) (layer "F.Cu") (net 2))
 (segment (start 148.59 90.32875) (end 167.64 90.32875) (width 0.2) (layer "F.Cu") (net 2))
 (segment (start 148.59 90.32875) (end 148.59 109.37875) (width 0.2) (layer "F.Cu") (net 2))
 (segment (start 174.175 111.318934) (end 172.234816 109.37875) (width 0.2) (layer "B.Cu") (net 2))
 (segment (start 174.175 92.268934) (end 172.234816 90.32875) (width 0.2) (layer "B.Cu") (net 2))
 (segment (start 172.234816 109.37875) (end 167.64 109.37875) (width 0.2) (layer "B.Cu") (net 2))
 (segment (start 153.184816 90.32875) (end 148.59 90.32875) (width 0.2) (layer "B.Cu") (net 2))
 (segment (start 155.075 96.65) (end 155.075 92.218934) (width 0.2) (layer "B.Cu") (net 2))
 (segment (start 174.175 96.65) (end 174.175 92.268934) (width 0.2) (layer "B.Cu") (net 2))
 (segment (start 155.075 115.65) (end 155.075 111.075) (width 0.2) (layer "B.Cu") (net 2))
 (segment (start 153.184816 71.27875) (end 148.59 71.27875) (width 0.2) (layer "B.Cu") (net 2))
 (segment (start 172.234816 90.32875) (end 167.64 90.32875) (width 0.2) (layer "B.Cu") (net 2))
 (segment (start 153.37875 109.37875) (end 148.59 109.37875) (width 0.2) (layer "B.Cu") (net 2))
 (segment (start 155.075 111.075) (end 153.37875 109.37875) (width 0.2) (layer "B.Cu") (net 2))
 (segment (start 155.1 73.193934) (end 153.184816 71.27875) (width 0.2) (layer "B.Cu") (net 2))
 (segment (start 155.075 92.218934) (end 153.184816 90.32875) (width 0.2) (layer "B.Cu") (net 2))
 (segment (start 174.175 115.65) (end 174.175 111.318934) (width 0.2) (layer "B.Cu") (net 2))
 (segment (start 155.1 77.6) (end 155.1 73.193934) (width 0.2) (layer "B.Cu") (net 2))
 (segment (start 160.369453 98.169453) (end 160.4 98.2) (width 0.2) (layer "F.Cu") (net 16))
 (segment (start 156.969453 98.169453) (end 160.369453 98.169453) (width 0.2) (layer "F.Cu") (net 16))
 (via (at 156.969453 98.169453) (size 0.6) (drill 0.3) (layers "F.Cu" "B.Cu") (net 16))
 (via (at 160.4 98.2) (size 0.6) (drill 0.3) (layers "F.Cu" "B.Cu") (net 16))
 (segment (start 155.075 98.15) (end 156.95 98.15) (width 0.2) (layer "B.Cu") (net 16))
 (segment (start 160.4 98.2) (end 161.95 96.65) (width 0.2) (layer "B.Cu") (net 16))
 (segment (start 161.95 96.65) (end 168.825 96.65) (width 0.2) (layer "B.Cu") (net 16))
 (segment (start 156.95 98.15) (end 156.969453 98.169453) (width 0.2) (layer "B.Cu") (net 16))
 (segment (start 175.201 90.981064) (end 175.201 97.439) (width 0.2) (layer "B.Cu") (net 19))
 (segment (start 149.725 112.62528) (end 146.82253 109.72281) (width 0.2) (layer "B.Cu") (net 19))
 (segment (start 149.725 115.65) (end 149.725 112.62528) (width 0.2) (layer "B.Cu") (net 19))
 (segment (start 175.201 97.439) (end 174.49 98.15) (width 0.2) (layer "B.Cu") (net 19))
 (segment (start 146.82253 109.164906) (end 167.618372 88.369064) (width 0.2) (layer "B.Cu") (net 19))
 (segment (start 174.49 98.15) (end 174.175 98.15) (width 0.2) (layer "B.Cu") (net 19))
 (segment (start 167.618372 88.369064) (end 172.589 88.369064) (width 0.2) (layer "B.Cu") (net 19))
 (segment (start 146.82253 109.72281) (end 146.82253 109.164906) (width 0.2) (layer "B.Cu") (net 19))
 (segment (start 172.589 88.369064) (end 175.201 90.981064) (width 0.2) (layer "B.Cu") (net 19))
 (segment (start 167.2 114.1) (end 167.3 114.1) (width 0.2) (layer "F.Cu") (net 18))
 (segment (start 165.8 115.5) (end 167.2 114.1) (width 0.2) (layer "F.Cu") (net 18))
 (via (at 165.8 115.5) (size 0.6) (drill 0.3) (layers "F.Cu" "B.Cu") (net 18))
 (via (at 167.3 114.1) (size 0.6) (drill 0.3) (layers "F.Cu" "B.Cu") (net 18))
 (segment (start 167.3 114.125) (end 168.825 115.65) (width 0.2) (layer "B.Cu") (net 18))
 (segment (start 165.8 115.5) (end 165.9 115.4) (width 0.2) (layer "B.Cu") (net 18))
 (segment (start 155.075 117.15) (end 164.15 117.15) (width 0.2) (layer "B.Cu") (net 18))
 (segment (start 164.15 117.15) (end 165.8 115.5) (width 0.2) (layer "B.Cu") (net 18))
 (segment (start 167.3 114.1) (end 167.3 114.125) (width 0.2) (layer "B.Cu") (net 18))
 (segment (start 128.465 77.28) (end 123.48 77.28) (width 0.2) (layer "B.Cu") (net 7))
 (segment (start 136.085 84.9) (end 128.465 77.28) (width 0.2) (layer "B.Cu") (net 7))
 (segment (start 123.48 74.74) (end 123.48 75.537) (width 0.2) (layer "F.Cu") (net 6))
 (segment (start 128.465 74.74) (end 123.48 74.74) (width 0.2) (layer "B.Cu") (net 6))
 (segment (start 138.625 84.9) (end 128.465 74.74) (width 0.2) (layer "B.Cu") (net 6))
 (segment (start 164.325 69.325) (end 164.325 71.31875) (width 0.2) (layer "F.Cu") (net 3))
 (segment (start 164.1 69.1) (end 164.325 69.325) (width 0.2) (layer "F.Cu") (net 3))
 (segment (start 161.717 63.517) (end 164.1 65.9) (width 0.2) (layer "F.Cu") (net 3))
 (segment (start 123.48 64.58) (end 124.543 63.517) (width 0.2) (layer "F.Cu") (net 3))
 (segment (start 124.543 63.517) (end 161.717 63.517) (width 0.2) (layer "F.Cu") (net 3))
 (via (at 164.1 69.1) (size 0.6) (drill 0.3) (layers "F.Cu" "B.Cu") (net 3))
 (via (at 164.1 65.9) (size 0.6) (drill 0.3) (layers "F.Cu" "B.Cu") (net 3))
 (segment (start 164.1 65.9) (end 164.1 69.1) (width 0.2) (layer "B.Cu") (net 3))
 (segment (start 123.48 67.12) (end 138.66 82.3) (width 0.2) (layer "F.Cu") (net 4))
 (segment (start 158.34375 82.3) (end 164.325 76.31875) (width 0.2) (layer "F.Cu") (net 4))
 (segment (start 150.2 82.3) (end 158.34375 82.3) (width 0.2) (layer "F.Cu") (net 4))
 (segment (start 138.66 82.3) (end 147.8 82.3) (width 0.2) (layer "F.Cu") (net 4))
 (via (at 147.8 82.3) (size 0.6) (drill 0.3) (layers "F.Cu" "B.Cu") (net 4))
 (via (at 150.2 82.3) (size 0.6) (drill 0.3) (layers "F.Cu" "B.Cu") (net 4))
 (segment (start 147.8 82.3) (end 150.2 82.3) (width 0.2) (layer "B.Cu") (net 4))
 (segment (start 139.783 73.263) (end 139.783 77.72031) (width 0.2) (layer "B.Cu") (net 12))
 (segment (start 138.11359 63.116) (end 149.31725 63.116) (width 0.2) (layer "B.Cu") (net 12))
 (segment (start 137.256 77.31931) (end 137.256 63.97359) (width 0.2) (layer "B.Cu") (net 12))
 (segment (start 138.72 72.2) (end 139.783 73.263) (width 0.2) (layer "B.Cu") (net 12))
 (segment (start 139.783 77.72031) (end 139.16031 78.343) (width 0.2) (layer "B.Cu") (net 12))
 (segment (start 139.16031 78.343) (end 138.27969 78.343) (width 0.2) (layer "B.Cu") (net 12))
 (segment (start 149.31725 63.116) (end 154.94 68.73875) (width 0.2) (layer "B.Cu") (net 12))
 (segment (start 138.27969 78.343) (end 137.256 77.31931) (width 0.2) (layer "B.Cu") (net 12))
 (segment (start 137.256 63.97359) (end 138.11359 63.116) (width 0.2) (layer "B.Cu") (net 12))
 (segment (start 153.28875 87.78875) (end 154.94 87.78875) (width 0.2) (layer "F.Cu") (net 11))
 (segment (start 150.2 84.7) (end 153.28875 87.78875) (width 0.2) (layer "F.Cu") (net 11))
 (segment (start 138.72 74.74) (end 130.037 66.057) (width 0.2) (layer "F.Cu") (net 11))
 (segment (start 121.389374 66.057) (end 121.128 66.318374) (width 0.2) (layer "F.Cu") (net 11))
 (segment (start 123.92031 68.183) (end 140.53731 84.8) (width 0.2) (layer "F.Cu") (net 11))
 (segment (start 140.53731 84.8) (end 147.8 84.8) (width 0.2) (layer "F.Cu") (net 11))
 (segment (start 121.389374 68.183) (end 123.92031 68.183) (width 0.2) (layer "F.Cu") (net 11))
 (segment (start 121.128 67.921626) (end 121.389374 68.183) (width 0.2) (layer "F.Cu") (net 11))
 (segment (start 121.128 66.318374) (end 121.128 67.921626) (width 0.2) (layer "F.Cu") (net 11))
 (segment (start 130.037 66.057) (end 121.389374 66.057) (width 0.2) (layer "F.Cu") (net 11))
 (via (at 147.8 84.8) (size 0.6) (drill 0.3) (layers "F.Cu" "B.Cu") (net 11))
 (via (at 150.2 84.7) (size 0.6) (drill 0.3) (layers "F.Cu" "B.Cu") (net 11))
 (segment (start 147.8 84.8) (end 150.1 84.8) (width 0.2) (layer "B.Cu") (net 11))
 (segment (start 150.1 84.8) (end 150.2 84.7) (width 0.2) (layer "B.Cu") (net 11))
 (segment (start 155.501 76.264) (end 155.501 73.027834) (width 0.2) (layer "B.Cu") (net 10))
 (segment (start 137.657 64.13969) (end 137.657 76.217) (width 0.2) (layer "B.Cu") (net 10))
 (segment (start 145.990166 63.517) (end 138.27969 63.517) (width 0.2) (layer "B.Cu") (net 10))
 (segment (start 167.02575 87.78875) (end 155.501 76.264) (width 0.2) (layer "B.Cu") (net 10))
 (segment (start 137.657 76.217) (end 138.72 77.28) (width 0.2) (layer "B.Cu") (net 10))
 (segment (start 138.27969 63.517) (end 137.657 64.13969) (width 0.2) (layer "B.Cu") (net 10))
 (segment (start 173.99 87.78875) (end 167.02575 87.78875) (width 0.2) (layer "B.Cu") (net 10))
 (segment (start 155.501 73.027834) (end 145.990166 63.517) (width 0.2) (layer "B.Cu") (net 10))
 (segment (start 149.170314 110.77975) (end 148.009686 110.77975) (width 0.2) (layer "F.Cu") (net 5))
 (segment (start 148.009686 110.77975) (end 124.543 87.313064) (width 0.2) (layer "F.Cu") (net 5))
 (segment (start 153.111314 106.83875) (end 149.170314 110.77975) (width 0.2) (layer "F.Cu") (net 5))
 (segment (start 124.543 87.313064) (end 124.543 73.263) (width 0.2) (layer "F.Cu") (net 5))
 (segment (start 124.543 73.263) (end 123.48 72.2) (width 0.2) (layer "F.Cu") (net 5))
 (segment (start 154.94 106.83875) (end 153.111314 106.83875) (width 0.2) (layer "F.Cu") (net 5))
 (segment (start 173.205184 106.83875) (end 173.99 106.83875) (width 0.2) (layer "F.Cu") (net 1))
 (segment (start 146.82253 113.11975) (end 147.81747 113.11975) (width 0.2) (layer "F.Cu") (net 1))
 (segment (start 147.81747 113.11975) (end 152.69747 108.23975) (width 0.2) (layer "F.Cu") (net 1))
 (segment (start 169.264184 110.77975) (end 173.205184 106.83875) (width 0.2) (layer "F.Cu") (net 1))
 (segment (start 121.128 71.398374) (end 121.128 87.42522) (width 0.2) (layer "F.Cu") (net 1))
 (segment (start 122.866374 69.66) (end 121.128 71.398374) (width 0.2) (layer "F.Cu") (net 1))
 (segment (start 121.128 87.42522) (end 146.82253 113.11975) (width 0.2) (layer "F.Cu") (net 1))
 (segment (start 164.519686 108.23975) (end 167.059686 110.77975) (width 0.2) (layer "F.Cu") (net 1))
 (segment (start 152.69747 108.23975) (end 164.519686 108.23975) (width 0.2) (layer "F.Cu") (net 1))
 (segment (start 123.48 69.66) (end 122.866374 69.66) (width 0.2) (layer "F.Cu") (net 1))
 (segment (start 167.059686 110.77975) (end 169.264184 110.77975) (width 0.2) (layer "F.Cu") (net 1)))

